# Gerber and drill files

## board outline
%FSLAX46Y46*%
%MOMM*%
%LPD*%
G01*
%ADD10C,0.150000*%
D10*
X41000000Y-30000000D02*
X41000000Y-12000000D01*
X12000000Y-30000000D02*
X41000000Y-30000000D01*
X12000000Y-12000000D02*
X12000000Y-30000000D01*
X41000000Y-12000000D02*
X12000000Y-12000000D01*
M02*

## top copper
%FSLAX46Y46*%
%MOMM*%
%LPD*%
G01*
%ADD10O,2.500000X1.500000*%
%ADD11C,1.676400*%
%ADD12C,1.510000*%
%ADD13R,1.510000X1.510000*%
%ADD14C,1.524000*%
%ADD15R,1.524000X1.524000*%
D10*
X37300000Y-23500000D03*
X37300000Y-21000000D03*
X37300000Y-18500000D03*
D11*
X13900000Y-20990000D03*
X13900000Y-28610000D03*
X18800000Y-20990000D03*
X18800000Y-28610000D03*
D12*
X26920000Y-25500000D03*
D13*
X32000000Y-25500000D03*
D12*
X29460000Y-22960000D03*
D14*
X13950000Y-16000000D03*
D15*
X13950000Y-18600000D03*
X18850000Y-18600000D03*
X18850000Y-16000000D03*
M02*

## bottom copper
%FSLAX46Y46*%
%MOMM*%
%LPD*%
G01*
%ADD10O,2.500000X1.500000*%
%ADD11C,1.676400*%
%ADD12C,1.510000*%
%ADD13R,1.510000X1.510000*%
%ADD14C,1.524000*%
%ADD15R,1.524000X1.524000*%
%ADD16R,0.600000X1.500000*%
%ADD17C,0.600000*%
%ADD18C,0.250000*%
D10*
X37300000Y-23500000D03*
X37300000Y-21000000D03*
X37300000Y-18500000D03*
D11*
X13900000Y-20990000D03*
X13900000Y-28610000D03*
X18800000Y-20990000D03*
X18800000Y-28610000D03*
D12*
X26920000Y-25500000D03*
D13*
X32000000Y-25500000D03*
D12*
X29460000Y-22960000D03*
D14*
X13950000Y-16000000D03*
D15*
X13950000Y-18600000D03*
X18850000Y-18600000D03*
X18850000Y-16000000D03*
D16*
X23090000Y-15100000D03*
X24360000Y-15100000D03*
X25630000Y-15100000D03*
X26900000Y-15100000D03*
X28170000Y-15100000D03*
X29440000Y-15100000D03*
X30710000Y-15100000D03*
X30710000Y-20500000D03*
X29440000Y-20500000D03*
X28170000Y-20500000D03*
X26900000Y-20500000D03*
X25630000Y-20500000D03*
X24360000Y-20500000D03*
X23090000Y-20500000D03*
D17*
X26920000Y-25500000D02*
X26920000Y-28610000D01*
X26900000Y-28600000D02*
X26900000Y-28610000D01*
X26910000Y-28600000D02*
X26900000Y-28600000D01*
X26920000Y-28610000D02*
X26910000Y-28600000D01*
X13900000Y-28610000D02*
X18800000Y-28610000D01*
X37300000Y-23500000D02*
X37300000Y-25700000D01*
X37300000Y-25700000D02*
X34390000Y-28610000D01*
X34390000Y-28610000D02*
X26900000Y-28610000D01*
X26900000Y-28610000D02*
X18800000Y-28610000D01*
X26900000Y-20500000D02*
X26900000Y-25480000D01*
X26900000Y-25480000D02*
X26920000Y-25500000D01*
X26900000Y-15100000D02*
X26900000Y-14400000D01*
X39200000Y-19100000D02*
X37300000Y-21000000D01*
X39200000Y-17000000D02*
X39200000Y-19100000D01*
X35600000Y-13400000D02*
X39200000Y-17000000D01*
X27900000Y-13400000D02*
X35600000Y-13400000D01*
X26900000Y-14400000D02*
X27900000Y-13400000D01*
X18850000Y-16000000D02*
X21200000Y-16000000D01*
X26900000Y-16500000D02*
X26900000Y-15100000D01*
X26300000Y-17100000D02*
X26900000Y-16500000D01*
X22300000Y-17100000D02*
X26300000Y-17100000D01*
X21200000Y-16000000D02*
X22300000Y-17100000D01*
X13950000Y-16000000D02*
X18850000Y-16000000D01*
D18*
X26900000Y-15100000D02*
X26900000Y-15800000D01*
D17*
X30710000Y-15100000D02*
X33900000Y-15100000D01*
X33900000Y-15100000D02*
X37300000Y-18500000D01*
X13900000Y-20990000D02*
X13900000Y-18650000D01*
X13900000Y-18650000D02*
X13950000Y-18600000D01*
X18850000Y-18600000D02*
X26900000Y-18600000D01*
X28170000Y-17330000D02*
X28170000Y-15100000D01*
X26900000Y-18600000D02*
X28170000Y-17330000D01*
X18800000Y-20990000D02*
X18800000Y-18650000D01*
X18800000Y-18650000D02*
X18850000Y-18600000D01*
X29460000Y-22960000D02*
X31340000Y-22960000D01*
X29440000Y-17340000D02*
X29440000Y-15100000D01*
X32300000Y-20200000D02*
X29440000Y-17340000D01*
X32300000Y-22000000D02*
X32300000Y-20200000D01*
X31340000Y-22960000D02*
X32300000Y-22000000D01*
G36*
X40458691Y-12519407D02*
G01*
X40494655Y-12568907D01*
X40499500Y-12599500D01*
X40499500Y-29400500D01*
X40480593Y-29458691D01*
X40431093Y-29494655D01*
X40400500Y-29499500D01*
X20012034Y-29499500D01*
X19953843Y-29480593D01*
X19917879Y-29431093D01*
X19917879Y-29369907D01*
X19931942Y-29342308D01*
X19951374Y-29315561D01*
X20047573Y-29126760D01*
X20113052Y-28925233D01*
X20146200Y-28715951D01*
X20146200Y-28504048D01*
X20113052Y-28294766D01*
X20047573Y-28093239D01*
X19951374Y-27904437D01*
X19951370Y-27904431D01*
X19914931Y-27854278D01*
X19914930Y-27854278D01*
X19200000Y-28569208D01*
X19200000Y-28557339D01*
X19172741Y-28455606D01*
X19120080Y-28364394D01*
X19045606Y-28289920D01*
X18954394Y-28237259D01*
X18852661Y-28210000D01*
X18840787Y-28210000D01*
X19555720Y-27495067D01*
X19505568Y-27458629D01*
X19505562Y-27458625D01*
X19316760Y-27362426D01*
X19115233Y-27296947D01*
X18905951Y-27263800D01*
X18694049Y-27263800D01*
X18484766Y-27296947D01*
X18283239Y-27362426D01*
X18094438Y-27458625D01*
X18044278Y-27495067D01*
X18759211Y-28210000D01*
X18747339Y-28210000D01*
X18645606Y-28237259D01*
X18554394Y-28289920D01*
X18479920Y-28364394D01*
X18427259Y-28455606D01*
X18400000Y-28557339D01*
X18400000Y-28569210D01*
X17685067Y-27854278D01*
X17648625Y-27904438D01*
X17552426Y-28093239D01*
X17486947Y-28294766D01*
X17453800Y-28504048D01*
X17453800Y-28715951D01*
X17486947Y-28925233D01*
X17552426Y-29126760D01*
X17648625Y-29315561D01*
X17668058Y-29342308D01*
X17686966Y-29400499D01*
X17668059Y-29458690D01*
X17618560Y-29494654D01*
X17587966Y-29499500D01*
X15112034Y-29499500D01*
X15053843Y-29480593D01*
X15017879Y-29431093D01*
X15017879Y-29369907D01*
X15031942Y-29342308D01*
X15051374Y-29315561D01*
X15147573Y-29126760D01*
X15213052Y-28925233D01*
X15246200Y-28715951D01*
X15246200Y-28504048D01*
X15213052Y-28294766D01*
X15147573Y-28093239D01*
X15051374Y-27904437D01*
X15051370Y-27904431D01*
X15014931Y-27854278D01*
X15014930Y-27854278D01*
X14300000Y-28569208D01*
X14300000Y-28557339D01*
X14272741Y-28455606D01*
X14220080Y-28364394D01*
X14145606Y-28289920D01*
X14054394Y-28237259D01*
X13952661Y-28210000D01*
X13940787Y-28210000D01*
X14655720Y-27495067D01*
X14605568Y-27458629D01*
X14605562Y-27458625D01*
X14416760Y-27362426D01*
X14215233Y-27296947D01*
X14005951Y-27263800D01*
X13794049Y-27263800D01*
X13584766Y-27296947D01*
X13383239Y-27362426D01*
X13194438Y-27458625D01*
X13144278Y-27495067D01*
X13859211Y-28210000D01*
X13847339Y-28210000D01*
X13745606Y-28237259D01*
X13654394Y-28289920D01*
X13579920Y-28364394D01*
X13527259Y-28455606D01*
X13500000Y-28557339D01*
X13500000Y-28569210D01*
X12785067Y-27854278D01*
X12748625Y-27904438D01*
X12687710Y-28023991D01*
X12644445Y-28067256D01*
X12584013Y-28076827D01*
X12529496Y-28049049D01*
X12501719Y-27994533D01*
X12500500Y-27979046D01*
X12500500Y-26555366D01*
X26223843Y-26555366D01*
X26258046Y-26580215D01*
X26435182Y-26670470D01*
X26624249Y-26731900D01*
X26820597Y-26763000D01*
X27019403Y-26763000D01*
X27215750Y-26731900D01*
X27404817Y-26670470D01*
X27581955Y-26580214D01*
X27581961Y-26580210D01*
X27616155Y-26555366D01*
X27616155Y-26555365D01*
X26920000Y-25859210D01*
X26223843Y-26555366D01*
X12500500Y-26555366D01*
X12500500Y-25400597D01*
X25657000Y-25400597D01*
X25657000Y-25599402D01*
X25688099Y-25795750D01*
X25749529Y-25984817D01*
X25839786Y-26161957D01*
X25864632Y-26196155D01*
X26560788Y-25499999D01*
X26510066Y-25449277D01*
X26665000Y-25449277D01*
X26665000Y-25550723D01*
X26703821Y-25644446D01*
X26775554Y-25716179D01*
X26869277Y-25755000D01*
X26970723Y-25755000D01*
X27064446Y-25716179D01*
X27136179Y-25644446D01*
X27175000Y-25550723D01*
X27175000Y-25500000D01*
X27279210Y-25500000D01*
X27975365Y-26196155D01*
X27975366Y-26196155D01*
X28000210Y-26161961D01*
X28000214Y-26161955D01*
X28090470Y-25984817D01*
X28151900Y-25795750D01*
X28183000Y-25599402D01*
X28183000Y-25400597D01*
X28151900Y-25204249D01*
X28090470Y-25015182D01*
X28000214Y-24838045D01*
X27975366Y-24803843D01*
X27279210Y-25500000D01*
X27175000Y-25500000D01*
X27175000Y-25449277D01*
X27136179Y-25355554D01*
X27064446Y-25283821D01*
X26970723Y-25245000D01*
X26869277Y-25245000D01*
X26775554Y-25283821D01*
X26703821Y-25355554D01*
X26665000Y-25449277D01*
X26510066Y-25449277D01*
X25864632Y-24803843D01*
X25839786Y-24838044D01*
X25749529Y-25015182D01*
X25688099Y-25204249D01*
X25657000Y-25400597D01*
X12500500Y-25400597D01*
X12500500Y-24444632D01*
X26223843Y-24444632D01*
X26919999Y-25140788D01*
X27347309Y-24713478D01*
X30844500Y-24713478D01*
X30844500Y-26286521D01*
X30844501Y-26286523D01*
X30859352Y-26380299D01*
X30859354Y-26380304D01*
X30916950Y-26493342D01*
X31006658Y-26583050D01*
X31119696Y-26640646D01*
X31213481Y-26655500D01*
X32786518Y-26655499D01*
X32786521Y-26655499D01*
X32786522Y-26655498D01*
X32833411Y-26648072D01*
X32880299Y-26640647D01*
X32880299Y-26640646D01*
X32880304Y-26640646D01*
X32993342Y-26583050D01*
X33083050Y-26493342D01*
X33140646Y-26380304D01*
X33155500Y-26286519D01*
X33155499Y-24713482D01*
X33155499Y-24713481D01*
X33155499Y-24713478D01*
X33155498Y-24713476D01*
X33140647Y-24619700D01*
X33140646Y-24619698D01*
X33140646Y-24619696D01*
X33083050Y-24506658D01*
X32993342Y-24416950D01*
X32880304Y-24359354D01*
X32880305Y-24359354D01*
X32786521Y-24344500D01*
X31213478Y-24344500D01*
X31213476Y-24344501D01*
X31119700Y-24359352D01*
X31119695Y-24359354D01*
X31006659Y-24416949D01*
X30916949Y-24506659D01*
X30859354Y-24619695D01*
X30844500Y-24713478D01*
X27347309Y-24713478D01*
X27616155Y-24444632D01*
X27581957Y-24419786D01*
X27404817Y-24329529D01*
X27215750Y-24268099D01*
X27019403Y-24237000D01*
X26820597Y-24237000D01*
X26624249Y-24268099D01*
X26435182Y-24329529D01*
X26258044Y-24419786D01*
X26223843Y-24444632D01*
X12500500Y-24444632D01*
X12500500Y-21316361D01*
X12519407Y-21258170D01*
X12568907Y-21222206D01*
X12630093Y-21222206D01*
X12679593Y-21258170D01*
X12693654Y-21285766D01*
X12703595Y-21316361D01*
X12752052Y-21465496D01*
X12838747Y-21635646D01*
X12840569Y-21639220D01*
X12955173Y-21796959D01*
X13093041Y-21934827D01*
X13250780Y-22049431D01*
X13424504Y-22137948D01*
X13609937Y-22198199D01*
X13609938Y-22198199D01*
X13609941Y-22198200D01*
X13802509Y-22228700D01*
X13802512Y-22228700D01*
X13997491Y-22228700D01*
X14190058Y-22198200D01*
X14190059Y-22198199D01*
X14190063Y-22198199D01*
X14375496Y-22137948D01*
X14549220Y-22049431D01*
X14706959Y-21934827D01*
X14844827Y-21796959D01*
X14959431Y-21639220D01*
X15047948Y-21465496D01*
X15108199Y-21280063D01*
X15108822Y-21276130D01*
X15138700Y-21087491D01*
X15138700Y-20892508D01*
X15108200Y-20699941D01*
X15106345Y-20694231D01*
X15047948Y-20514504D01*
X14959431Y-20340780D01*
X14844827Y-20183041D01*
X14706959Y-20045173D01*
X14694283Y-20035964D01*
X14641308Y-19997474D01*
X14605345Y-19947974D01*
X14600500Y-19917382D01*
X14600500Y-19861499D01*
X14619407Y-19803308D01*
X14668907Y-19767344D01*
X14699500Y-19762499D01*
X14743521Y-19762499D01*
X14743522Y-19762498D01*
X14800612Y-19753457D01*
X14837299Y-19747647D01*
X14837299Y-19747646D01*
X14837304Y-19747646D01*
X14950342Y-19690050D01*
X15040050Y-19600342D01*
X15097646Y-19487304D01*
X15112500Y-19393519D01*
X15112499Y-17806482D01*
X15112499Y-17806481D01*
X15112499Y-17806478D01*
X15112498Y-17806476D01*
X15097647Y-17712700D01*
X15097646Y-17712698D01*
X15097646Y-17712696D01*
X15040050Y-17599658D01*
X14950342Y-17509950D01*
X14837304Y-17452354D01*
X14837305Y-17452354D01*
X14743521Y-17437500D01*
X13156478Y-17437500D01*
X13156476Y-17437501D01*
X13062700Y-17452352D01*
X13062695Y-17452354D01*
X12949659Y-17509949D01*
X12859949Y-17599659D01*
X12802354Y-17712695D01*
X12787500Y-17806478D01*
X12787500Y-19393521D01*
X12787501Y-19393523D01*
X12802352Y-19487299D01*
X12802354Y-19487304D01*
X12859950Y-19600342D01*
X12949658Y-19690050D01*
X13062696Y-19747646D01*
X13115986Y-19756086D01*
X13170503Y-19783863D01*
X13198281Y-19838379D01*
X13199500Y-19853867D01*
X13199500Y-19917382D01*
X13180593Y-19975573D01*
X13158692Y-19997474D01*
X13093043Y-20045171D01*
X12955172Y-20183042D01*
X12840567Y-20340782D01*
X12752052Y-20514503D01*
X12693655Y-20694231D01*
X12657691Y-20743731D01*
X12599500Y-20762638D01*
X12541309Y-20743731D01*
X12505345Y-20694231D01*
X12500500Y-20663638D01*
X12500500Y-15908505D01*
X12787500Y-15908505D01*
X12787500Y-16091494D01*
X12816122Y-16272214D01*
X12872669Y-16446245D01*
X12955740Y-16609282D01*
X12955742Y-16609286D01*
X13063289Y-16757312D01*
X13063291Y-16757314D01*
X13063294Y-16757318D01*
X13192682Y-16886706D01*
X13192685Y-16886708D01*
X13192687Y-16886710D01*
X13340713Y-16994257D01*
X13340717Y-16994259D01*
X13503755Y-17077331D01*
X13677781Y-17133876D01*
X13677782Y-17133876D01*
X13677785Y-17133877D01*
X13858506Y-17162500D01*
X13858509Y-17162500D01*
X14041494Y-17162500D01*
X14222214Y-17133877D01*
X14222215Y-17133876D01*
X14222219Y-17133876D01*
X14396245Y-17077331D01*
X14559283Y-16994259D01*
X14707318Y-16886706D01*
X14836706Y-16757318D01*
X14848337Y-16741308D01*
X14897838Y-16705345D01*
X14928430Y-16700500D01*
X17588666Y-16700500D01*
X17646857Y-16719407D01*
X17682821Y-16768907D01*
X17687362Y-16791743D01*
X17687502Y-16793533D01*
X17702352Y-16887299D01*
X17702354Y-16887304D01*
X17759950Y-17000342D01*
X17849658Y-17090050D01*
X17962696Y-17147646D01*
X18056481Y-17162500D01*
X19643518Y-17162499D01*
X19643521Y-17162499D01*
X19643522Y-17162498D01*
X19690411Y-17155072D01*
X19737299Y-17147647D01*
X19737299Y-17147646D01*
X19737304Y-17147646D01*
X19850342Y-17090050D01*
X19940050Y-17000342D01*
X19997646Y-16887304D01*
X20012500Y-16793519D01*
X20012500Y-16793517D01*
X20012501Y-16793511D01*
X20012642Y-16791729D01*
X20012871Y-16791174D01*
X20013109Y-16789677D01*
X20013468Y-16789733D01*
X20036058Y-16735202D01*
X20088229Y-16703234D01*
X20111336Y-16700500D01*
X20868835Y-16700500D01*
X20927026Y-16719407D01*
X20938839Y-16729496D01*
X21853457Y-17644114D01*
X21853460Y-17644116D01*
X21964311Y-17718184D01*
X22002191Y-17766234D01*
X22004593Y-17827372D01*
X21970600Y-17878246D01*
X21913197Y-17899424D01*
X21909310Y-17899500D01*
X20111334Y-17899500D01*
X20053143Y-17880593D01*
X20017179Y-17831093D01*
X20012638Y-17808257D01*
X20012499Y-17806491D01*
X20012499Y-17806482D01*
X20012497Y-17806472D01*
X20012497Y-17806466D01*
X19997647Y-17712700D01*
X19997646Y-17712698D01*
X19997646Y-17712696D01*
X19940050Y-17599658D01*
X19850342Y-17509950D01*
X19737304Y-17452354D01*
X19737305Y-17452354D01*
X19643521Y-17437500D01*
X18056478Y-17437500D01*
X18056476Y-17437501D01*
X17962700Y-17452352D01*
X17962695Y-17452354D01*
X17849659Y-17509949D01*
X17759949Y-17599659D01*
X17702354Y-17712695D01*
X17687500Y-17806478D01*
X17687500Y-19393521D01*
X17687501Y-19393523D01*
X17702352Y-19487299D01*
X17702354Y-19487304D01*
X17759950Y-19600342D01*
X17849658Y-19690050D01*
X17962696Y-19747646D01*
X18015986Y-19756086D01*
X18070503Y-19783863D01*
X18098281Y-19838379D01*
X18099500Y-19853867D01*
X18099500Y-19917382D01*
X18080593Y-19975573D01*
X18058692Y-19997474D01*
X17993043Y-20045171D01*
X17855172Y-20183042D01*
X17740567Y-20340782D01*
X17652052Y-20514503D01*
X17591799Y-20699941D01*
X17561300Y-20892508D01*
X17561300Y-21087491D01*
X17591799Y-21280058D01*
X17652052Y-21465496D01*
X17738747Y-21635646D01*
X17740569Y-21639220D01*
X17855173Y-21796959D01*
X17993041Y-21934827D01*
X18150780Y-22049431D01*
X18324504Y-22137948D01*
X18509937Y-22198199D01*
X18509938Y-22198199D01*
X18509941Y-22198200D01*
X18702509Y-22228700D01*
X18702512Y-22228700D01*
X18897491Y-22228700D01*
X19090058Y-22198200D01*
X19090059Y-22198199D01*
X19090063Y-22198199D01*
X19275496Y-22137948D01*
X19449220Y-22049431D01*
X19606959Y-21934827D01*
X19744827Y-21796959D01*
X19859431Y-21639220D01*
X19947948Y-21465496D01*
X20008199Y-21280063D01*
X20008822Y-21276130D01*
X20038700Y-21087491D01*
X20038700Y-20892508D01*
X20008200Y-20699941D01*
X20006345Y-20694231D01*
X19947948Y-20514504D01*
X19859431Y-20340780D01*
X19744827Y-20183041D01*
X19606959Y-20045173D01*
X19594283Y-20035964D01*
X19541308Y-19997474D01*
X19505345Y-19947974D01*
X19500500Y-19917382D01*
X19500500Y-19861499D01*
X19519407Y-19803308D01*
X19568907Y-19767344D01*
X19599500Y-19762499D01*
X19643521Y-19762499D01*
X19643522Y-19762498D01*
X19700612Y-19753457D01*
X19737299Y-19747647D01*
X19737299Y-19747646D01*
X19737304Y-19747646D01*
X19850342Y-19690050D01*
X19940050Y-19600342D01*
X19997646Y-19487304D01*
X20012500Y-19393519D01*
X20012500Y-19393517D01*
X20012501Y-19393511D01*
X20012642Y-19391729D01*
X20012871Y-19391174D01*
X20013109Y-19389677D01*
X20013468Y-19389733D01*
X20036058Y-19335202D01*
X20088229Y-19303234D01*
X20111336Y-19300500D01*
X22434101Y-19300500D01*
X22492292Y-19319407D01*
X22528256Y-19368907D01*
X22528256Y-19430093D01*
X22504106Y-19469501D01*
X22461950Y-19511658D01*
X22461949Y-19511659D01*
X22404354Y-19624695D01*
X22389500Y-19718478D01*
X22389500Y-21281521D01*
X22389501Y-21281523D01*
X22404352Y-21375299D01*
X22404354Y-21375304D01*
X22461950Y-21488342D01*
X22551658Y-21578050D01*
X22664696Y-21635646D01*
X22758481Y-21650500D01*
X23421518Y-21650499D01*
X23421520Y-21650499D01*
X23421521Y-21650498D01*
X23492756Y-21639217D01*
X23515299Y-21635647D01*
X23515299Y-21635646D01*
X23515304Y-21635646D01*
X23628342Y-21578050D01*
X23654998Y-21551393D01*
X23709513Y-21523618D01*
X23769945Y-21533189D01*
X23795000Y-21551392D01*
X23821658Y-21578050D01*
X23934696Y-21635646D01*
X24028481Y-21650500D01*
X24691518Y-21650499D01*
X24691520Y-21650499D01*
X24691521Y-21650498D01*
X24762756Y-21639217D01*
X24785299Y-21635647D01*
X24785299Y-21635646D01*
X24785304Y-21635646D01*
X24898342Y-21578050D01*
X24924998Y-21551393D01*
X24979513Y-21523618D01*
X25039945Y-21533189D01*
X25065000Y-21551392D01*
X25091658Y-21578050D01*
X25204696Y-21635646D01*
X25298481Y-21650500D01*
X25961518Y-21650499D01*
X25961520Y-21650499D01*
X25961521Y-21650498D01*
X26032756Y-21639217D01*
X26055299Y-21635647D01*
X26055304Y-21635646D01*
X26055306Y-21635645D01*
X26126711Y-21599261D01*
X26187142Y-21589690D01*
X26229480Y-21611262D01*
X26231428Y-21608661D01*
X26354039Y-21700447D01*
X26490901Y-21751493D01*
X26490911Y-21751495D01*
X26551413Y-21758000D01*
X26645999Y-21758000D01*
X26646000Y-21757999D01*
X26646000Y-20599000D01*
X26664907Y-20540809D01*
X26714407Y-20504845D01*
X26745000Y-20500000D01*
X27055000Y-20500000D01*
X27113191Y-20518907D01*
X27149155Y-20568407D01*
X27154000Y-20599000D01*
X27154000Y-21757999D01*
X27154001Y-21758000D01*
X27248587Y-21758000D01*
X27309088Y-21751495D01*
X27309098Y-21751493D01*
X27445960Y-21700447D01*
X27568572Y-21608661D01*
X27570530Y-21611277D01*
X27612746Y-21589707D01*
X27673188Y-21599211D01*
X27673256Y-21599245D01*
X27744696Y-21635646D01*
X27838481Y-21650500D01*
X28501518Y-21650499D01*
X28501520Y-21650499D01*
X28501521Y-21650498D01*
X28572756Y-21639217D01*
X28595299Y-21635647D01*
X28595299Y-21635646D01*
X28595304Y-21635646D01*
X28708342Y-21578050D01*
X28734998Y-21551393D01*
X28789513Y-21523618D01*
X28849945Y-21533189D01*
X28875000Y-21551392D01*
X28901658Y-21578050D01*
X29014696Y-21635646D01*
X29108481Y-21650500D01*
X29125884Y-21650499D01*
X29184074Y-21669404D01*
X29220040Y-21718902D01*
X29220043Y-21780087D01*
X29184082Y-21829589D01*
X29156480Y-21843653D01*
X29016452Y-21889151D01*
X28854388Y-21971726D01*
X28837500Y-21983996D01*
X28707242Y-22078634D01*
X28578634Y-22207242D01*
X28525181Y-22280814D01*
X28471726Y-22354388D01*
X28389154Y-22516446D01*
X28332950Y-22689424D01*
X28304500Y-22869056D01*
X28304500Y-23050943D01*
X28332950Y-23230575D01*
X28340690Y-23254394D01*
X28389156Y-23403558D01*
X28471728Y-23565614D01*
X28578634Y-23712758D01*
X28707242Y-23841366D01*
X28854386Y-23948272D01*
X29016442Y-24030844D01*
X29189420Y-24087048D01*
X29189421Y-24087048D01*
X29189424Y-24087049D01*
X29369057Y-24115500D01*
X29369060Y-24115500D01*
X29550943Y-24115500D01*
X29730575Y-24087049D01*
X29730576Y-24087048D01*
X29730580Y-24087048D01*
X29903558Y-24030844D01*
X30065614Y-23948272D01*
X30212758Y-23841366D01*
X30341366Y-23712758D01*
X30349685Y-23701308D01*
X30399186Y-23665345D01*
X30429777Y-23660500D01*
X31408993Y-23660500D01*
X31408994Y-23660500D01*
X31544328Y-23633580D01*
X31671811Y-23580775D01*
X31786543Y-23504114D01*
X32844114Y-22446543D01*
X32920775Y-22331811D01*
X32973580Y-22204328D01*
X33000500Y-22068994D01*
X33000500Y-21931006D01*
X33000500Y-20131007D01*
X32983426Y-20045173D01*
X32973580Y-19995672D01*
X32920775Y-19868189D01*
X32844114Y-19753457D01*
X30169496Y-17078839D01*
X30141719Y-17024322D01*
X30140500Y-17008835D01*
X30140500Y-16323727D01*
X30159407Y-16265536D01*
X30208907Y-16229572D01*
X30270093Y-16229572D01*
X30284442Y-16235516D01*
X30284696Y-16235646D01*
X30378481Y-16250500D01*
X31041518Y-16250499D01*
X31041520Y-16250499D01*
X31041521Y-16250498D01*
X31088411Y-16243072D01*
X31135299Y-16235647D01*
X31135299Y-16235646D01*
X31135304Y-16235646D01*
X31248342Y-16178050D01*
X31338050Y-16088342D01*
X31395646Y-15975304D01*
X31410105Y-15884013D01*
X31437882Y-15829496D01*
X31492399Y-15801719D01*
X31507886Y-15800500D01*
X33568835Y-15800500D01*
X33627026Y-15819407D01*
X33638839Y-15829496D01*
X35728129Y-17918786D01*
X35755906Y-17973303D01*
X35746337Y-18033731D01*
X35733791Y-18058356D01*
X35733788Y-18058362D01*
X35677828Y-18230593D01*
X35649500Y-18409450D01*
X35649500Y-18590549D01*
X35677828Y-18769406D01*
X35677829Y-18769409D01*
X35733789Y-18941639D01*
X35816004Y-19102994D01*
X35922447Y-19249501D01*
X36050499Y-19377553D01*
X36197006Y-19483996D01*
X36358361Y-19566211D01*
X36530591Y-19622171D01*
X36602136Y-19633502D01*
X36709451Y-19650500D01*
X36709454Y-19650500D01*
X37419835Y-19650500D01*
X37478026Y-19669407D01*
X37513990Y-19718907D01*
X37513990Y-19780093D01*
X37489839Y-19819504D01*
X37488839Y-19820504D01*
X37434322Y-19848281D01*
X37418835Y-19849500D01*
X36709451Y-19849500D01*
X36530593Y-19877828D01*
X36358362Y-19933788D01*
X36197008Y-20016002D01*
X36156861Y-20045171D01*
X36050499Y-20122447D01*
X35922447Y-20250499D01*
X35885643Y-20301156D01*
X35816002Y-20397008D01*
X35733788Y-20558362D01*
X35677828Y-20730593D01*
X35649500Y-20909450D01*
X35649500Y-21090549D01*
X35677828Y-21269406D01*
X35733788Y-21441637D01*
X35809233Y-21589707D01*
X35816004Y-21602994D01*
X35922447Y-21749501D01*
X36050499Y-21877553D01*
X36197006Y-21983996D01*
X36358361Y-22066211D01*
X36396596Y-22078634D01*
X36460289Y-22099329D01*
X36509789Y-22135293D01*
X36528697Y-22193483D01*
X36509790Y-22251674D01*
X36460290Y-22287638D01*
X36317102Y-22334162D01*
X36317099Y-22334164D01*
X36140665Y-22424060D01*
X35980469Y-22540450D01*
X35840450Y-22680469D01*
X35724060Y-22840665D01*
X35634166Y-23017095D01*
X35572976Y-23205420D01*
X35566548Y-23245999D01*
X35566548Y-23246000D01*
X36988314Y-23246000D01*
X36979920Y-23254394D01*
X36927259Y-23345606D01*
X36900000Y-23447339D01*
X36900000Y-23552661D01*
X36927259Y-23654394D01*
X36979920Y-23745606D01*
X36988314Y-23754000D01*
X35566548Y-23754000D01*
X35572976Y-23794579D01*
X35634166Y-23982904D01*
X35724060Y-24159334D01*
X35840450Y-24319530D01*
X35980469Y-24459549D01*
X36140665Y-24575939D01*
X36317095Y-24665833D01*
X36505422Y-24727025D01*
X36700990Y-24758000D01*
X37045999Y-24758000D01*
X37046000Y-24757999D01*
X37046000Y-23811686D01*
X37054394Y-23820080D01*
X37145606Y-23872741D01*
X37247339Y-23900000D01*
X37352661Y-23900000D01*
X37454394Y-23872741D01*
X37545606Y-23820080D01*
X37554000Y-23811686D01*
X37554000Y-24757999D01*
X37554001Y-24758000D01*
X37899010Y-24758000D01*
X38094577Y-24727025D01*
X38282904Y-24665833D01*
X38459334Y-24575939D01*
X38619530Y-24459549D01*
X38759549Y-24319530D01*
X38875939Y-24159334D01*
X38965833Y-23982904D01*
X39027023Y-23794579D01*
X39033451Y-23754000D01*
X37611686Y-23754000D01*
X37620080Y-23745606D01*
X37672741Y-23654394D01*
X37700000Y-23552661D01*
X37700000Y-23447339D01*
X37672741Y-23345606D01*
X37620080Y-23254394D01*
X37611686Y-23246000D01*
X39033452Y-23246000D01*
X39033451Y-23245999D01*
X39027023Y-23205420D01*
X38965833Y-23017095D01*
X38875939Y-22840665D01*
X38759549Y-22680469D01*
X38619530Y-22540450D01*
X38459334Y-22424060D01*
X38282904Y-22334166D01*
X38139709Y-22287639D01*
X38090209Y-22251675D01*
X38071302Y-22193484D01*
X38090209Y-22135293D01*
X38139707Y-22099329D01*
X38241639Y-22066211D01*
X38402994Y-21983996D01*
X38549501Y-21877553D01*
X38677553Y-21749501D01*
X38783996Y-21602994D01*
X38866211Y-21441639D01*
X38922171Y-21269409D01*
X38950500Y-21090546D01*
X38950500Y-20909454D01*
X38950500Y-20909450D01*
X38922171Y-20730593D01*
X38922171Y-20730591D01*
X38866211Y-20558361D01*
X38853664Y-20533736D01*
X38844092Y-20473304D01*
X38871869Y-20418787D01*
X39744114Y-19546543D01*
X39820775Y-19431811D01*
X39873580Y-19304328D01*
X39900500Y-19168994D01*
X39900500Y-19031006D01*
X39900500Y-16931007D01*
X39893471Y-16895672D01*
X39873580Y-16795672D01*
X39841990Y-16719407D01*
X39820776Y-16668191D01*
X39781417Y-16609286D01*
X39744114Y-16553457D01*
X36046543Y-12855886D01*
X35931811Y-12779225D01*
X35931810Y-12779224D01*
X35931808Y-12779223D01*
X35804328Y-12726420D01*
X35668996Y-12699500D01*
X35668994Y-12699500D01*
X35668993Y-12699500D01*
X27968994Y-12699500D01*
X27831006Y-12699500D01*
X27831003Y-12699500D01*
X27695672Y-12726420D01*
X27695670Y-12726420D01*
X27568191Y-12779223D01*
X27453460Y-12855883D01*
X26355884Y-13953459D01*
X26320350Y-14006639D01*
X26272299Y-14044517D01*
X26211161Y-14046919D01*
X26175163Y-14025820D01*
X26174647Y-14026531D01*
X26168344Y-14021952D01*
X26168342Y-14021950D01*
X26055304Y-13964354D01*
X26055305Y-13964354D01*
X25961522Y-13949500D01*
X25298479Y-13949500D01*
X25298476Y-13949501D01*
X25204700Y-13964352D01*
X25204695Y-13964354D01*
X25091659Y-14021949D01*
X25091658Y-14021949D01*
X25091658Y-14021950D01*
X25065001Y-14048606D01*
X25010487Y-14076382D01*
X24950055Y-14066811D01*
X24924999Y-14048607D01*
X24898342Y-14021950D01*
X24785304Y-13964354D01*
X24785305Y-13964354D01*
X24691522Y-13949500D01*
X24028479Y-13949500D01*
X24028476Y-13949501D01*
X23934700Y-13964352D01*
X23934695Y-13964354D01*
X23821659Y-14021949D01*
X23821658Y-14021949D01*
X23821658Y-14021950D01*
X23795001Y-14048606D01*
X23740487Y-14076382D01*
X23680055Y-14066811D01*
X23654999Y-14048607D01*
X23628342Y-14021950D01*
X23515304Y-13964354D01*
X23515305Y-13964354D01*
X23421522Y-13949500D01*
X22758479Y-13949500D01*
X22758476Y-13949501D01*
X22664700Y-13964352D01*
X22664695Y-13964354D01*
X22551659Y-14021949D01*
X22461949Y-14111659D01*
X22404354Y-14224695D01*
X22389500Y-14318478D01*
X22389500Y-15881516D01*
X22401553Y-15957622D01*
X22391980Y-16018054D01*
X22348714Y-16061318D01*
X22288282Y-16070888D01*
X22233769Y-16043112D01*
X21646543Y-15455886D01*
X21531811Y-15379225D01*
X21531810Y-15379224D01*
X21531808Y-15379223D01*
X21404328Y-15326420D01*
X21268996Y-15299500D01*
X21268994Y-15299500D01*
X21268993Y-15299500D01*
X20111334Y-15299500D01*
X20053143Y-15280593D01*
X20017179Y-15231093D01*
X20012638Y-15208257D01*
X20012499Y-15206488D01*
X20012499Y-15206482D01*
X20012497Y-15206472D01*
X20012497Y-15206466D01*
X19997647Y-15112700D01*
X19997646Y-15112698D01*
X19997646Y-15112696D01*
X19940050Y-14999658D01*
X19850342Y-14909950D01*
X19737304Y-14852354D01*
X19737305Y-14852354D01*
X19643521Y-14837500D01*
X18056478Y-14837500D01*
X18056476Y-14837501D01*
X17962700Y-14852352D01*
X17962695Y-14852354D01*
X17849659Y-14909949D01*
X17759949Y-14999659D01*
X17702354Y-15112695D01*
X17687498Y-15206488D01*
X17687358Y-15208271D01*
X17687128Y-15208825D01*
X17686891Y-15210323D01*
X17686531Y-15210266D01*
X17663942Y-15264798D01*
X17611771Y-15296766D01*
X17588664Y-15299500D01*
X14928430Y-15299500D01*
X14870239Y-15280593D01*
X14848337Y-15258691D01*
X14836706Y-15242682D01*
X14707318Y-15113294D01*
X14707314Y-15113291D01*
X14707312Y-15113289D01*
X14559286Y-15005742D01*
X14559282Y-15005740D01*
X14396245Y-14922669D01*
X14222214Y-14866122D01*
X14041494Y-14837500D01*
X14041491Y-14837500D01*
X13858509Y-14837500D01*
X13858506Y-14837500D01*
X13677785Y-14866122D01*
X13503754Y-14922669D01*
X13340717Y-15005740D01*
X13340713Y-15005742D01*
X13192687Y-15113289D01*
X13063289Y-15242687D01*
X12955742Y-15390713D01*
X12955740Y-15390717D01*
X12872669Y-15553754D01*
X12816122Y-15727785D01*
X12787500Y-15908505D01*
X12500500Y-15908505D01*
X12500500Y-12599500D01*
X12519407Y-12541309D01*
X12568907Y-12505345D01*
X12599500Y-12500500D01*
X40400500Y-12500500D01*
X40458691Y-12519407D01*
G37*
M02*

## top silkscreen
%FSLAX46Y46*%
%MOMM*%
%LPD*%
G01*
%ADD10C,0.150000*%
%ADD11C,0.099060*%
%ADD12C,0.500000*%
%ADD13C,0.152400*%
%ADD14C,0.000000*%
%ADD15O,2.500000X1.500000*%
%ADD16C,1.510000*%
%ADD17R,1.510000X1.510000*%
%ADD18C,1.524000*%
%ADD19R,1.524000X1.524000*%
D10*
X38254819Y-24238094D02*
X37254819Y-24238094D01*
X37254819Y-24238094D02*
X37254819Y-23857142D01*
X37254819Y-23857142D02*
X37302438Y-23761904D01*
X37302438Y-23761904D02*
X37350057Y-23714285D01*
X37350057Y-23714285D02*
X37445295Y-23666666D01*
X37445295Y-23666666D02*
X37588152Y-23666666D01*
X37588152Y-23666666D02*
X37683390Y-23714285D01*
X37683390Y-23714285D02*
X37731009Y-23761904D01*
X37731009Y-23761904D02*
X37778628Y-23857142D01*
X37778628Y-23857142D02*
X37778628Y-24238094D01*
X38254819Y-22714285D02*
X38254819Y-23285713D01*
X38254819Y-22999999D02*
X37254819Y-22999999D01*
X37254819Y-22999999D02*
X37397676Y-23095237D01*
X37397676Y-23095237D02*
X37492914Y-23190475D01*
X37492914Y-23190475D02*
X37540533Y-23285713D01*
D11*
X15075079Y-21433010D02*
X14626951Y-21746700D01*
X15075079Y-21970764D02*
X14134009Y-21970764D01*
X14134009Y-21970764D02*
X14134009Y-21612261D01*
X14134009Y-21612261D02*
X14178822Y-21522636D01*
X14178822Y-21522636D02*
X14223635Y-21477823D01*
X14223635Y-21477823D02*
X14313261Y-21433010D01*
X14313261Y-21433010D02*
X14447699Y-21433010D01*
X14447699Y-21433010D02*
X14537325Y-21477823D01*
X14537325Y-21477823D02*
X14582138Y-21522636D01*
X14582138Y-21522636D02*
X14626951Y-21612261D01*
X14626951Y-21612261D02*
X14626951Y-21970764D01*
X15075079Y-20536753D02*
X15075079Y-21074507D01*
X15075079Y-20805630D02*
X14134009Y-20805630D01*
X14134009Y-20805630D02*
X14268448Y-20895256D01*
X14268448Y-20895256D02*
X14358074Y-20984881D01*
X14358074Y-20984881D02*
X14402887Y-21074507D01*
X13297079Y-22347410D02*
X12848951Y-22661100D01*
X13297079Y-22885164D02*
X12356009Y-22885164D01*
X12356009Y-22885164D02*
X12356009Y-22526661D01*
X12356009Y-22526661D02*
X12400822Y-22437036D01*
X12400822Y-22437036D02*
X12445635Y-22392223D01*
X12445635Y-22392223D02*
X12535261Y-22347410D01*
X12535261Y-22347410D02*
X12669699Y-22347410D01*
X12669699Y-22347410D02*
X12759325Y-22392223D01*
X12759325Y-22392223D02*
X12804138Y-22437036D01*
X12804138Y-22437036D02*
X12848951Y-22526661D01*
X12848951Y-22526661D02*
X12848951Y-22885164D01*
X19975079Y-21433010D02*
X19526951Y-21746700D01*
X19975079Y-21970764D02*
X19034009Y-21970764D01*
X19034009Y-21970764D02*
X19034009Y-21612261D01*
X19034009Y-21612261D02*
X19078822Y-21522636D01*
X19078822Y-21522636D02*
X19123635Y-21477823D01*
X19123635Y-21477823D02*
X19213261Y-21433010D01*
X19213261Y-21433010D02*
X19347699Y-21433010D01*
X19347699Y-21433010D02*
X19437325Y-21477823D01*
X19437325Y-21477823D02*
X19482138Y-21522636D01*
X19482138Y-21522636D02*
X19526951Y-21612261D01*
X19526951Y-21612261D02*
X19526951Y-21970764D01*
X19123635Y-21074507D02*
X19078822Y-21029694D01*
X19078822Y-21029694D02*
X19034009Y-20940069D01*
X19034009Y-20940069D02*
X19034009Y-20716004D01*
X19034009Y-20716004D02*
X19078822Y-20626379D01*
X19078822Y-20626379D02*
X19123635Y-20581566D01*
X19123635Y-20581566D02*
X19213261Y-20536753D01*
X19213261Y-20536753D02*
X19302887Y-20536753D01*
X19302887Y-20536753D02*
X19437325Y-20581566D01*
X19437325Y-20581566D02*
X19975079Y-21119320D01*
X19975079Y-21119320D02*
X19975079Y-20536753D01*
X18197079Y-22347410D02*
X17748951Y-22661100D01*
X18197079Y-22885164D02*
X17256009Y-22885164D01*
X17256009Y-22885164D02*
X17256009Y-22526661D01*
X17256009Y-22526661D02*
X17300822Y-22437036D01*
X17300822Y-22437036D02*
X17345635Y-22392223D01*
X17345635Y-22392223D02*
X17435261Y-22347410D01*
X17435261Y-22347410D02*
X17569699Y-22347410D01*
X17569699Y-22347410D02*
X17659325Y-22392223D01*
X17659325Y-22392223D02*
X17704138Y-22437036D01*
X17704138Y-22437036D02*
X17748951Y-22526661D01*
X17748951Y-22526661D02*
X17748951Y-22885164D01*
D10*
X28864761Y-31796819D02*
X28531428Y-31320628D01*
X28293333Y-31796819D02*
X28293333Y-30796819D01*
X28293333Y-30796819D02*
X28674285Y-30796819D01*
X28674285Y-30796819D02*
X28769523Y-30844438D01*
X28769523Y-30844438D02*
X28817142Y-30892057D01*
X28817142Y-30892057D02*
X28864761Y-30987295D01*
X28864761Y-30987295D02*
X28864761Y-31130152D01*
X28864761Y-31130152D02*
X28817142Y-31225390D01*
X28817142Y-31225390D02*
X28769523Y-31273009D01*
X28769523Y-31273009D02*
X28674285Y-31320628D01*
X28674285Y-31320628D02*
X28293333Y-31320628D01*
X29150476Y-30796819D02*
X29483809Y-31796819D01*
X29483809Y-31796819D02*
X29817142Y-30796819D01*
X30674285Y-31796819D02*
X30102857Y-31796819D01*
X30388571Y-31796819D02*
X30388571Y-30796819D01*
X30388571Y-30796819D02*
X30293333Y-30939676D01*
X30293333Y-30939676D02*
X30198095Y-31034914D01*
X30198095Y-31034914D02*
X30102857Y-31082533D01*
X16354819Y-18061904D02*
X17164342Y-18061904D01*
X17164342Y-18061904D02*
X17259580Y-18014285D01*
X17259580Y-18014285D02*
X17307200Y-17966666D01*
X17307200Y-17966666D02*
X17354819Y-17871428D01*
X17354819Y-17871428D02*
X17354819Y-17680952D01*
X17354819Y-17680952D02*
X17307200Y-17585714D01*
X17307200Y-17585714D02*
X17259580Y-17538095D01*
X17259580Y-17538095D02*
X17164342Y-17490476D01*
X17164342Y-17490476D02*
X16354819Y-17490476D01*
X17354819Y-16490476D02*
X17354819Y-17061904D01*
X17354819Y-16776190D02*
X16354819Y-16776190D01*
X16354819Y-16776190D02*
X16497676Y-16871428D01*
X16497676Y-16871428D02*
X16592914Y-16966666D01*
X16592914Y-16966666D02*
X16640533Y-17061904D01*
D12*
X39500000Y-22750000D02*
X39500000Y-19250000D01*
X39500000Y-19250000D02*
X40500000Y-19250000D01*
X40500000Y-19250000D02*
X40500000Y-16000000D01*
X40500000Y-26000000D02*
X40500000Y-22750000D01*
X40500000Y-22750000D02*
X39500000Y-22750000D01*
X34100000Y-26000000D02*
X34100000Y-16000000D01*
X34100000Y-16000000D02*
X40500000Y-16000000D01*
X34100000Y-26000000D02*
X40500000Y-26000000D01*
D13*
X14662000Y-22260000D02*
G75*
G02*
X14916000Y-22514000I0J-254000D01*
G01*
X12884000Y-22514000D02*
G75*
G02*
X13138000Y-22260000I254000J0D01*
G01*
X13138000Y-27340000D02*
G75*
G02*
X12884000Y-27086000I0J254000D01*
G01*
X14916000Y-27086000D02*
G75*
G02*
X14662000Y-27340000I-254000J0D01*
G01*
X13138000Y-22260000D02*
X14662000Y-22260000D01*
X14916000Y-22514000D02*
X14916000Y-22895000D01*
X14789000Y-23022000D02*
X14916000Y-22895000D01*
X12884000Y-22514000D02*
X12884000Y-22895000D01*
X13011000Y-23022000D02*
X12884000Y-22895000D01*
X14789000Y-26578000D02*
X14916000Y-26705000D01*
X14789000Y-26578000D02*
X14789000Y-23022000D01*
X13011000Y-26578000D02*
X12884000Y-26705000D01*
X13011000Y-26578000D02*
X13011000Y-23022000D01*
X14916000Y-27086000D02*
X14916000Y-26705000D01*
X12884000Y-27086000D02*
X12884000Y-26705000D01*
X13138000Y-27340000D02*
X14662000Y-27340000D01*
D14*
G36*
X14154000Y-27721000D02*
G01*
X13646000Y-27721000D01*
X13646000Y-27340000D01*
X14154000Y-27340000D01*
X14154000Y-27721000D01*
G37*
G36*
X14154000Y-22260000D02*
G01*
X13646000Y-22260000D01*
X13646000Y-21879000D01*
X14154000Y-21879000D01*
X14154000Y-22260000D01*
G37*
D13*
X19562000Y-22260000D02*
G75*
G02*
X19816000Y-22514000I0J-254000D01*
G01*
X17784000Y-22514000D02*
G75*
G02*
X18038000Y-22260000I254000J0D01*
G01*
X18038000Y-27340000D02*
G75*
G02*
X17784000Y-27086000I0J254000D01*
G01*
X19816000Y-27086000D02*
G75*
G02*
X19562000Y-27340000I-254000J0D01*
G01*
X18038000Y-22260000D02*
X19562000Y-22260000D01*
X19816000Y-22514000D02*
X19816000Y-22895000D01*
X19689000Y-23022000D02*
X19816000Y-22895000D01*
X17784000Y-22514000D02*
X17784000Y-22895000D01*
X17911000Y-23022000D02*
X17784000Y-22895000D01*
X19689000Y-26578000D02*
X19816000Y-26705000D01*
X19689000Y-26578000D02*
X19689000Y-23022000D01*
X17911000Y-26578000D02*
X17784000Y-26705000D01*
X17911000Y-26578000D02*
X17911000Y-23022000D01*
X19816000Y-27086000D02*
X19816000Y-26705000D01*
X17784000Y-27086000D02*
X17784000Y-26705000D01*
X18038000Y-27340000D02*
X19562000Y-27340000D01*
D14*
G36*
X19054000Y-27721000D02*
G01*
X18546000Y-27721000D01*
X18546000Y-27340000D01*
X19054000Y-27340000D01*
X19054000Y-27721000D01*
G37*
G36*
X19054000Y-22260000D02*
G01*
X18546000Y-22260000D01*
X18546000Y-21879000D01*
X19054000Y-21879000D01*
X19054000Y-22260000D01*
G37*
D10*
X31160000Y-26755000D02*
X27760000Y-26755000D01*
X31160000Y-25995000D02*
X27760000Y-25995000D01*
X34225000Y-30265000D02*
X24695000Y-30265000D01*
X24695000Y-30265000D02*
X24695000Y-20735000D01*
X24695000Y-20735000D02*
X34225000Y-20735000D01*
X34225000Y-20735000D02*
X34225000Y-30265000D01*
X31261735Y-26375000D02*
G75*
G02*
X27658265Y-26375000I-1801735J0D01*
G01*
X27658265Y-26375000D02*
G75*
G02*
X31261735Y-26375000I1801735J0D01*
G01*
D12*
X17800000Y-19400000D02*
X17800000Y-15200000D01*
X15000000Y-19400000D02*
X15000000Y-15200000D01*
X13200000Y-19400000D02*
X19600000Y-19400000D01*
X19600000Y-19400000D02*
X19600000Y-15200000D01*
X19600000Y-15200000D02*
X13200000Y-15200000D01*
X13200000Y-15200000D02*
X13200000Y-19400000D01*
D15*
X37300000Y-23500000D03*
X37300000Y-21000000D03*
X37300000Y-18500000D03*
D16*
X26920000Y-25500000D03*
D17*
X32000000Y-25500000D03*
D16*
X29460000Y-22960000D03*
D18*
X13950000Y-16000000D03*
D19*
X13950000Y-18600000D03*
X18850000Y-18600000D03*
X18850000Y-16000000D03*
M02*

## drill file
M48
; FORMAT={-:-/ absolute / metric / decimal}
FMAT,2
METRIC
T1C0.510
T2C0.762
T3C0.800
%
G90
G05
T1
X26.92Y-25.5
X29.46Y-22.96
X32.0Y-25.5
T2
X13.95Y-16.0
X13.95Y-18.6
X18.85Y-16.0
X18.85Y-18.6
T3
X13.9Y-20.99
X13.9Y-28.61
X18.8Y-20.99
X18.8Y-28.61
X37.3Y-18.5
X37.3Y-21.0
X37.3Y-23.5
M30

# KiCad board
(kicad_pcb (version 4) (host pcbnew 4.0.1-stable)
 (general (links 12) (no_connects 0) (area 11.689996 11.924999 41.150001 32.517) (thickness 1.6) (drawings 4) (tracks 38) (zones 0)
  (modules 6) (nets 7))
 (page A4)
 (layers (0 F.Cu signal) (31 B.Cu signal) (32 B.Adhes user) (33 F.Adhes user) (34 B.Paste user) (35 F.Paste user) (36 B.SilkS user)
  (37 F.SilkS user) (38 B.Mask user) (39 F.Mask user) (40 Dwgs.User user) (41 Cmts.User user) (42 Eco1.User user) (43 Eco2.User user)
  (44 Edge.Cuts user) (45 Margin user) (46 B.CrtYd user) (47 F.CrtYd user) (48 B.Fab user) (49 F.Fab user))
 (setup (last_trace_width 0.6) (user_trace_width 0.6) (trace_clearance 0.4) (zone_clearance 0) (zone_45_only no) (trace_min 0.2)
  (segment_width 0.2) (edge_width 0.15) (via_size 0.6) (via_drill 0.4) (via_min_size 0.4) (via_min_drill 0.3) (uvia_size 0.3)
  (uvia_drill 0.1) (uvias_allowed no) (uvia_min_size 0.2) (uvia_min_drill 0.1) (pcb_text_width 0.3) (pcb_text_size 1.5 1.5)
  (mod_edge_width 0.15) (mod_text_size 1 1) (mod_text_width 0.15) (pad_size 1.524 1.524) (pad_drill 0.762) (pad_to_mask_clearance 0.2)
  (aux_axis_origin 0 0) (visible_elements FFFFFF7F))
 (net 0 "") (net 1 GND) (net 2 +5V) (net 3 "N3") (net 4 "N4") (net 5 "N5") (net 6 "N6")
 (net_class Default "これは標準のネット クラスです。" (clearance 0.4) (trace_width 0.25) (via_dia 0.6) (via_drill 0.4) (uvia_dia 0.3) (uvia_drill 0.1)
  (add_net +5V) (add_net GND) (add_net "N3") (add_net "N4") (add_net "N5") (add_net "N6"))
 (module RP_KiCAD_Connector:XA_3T (layer F.Cu) (at 37.3 23.5 90)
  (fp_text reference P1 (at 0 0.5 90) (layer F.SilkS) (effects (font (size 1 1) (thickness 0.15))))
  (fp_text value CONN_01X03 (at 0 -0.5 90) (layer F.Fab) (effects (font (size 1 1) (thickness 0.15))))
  (fp_line (start 0.75 2.2) (end 4.25 2.2) (layer F.SilkS) (width 0.5))
  (fp_line (start 4.25 2.2) (end 4.25 3.2) (layer F.SilkS) (width 0.5))
  (fp_line (start 4.25 3.2) (end 7.5 3.2) (layer F.SilkS) (width 0.5))
  (fp_line (start -2.5 3.2) (end 0.75 3.2) (layer F.SilkS) (width 0.5))
  (fp_line (start 0.75 3.2) (end 0.75 2.2) (layer F.SilkS) (width 0.5))
  (fp_line (start -2.5 -3.2) (end 7.5 -3.2) (layer F.SilkS) (width 0.5))
  (fp_line (start 7.5 -3.2) (end 7.5 3.2) (layer F.SilkS) (width 0.5))
  (fp_line (start -2.5 -3.2) (end -2.5 3.2) (layer F.SilkS) (width 0.5))
  (pad 1 thru_hole oval (at 0 0 90) (size 1.5 2.5) (drill 0.8) (layers *.Cu *.Mask F.SilkS) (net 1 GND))
  (pad 2 thru_hole oval (at 2.5 0 90) (size 1.5 2.5) (drill 0.8) (layers *.Cu *.Mask F.SilkS) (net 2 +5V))
  (pad 3 thru_hole oval (at 5 0 90) (size 1.5 2.5) (drill 0.8) (layers *.Cu *.Mask F.SilkS) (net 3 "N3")))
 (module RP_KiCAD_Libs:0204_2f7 (layer F.Cu) (at 13.9 24.8 270)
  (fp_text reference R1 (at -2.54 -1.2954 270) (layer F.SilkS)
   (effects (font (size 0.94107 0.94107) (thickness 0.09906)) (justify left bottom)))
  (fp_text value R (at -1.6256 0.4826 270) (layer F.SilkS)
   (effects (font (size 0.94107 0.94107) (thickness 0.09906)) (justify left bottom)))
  (fp_arc (start -2.286 -0.762) (end -2.54 -0.762) (angle 90) (layer F.SilkS) (width 0.1524))
  (fp_arc (start -2.286 0.762) (end -2.54 0.762) (angle -90) (layer F.SilkS) (width 0.1524))
  (fp_arc (start 2.286 0.762) (end 2.286 1.016) (angle -90) (layer F.SilkS) (width 0.1524))
  (fp_arc (start 2.286 -0.762) (end 2.286 -1.016) (angle 90) (layer F.SilkS) (width 0.1524))
  (fp_line (start -2.54 0.762) (end -2.54 -0.762) (layer F.SilkS) (width 0.1524))
  (fp_line (start -2.286 -1.016) (end -1.905 -1.016) (layer F.SilkS) (width 0.1524))
  (fp_line (start -1.778 -0.889) (end -1.905 -1.016) (layer F.SilkS) (width 0.1524))
  (fp_line (start -2.286 1.016) (end -1.905 1.016) (layer F.SilkS) (width 0.1524))
  (fp_line (start -1.778 0.889) (end -1.905 1.016) (layer F.SilkS) (width 0.1524))
  (fp_line (start 1.778 -0.889) (end 1.905 -1.016) (layer F.SilkS) (width 0.1524))
  (fp_line (start 1.778 -0.889) (end -1.778 -0.889) (layer F.SilkS) (width 0.1524))
  (fp_line (start 1.778 0.889) (end 1.905 1.016) (layer F.SilkS) (width 0.1524))
  (fp_line (start 1.778 0.889) (end -1.778 0.889) (layer F.SilkS) (width 0.1524))
  (fp_line (start 2.286 -1.016) (end 1.905 -1.016) (layer F.SilkS) (width 0.1524))
  (fp_line (start 2.286 1.016) (end 1.905 1.016) (layer F.SilkS) (width 0.1524))
  (fp_line (start 2.54 0.762) (end 2.54 -0.762) (layer F.SilkS) (width 0.1524))
  (fp_poly (pts (xy 2.54 0.254) (xy 2.921 0.254) (xy 2.921 -0.254) (xy 2.54 -0.254)) (layer F.SilkS) (width 0))
  (fp_poly (pts (xy -2.921 0.254) (xy -2.54 0.254) (xy -2.54 -0.254) (xy -2.921 -0.254)) (layer F.SilkS) (width 0))
  (pad 1 thru_hole circle (at -3.81 0 270) (size 1.6764 1.6764) (drill 0.8) (layers *.Cu *.Mask) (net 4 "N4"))
  (pad 2 thru_hole circle (at 3.81 0 270) (size 1.6764 1.6764) (drill 0.8) (layers *.Cu *.Mask) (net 1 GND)))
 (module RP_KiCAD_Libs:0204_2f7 (layer F.Cu) (at 18.8 24.8 270)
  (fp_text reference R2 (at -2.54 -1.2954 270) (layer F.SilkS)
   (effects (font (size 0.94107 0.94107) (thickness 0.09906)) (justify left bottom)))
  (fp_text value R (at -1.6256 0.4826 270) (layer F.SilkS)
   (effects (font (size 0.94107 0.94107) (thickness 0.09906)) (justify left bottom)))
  (fp_arc (start -2.286 -0.762) (end -2.54 -0.762) (angle 90) (layer F.SilkS) (width 0.1524))
  (fp_arc (start -2.286 0.762) (end -2.54 0.762) (angle -90) (layer F.SilkS) (width 0.1524))
  (fp_arc (start 2.286 0.762) (end 2.286 1.016) (angle -90) (layer F.SilkS) (width 0.1524))
  (fp_arc (start 2.286 -0.762) (end 2.286 -1.016) (angle 90) (layer F.SilkS) (width 0.1524))
  (fp_line (start -2.54 0.762) (end -2.54 -0.762) (layer F.SilkS) (width 0.1524))
  (fp_line (start -2.286 -1.016) (end -1.905 -1.016) (layer F.SilkS) (width 0.1524))
  (fp_line (start -1.778 -0.889) (end -1.905 -1.016) (layer F.SilkS) (width 0.1524))
  (fp_line (start -2.286 1.016) (end -1.905 1.016) (layer F.SilkS) (width 0.1524))
  (fp_line (start -1.778 0.889) (end -1.905 1.016) (layer F.SilkS) (width 0.1524))
  (fp_line (start 1.778 -0.889) (end 1.905 -1.016) (layer F.SilkS) (width 0.1524))
  (fp_line (start 1.778 -0.889) (end -1.778 -0.889) (layer F.SilkS) (width 0.1524))
  (fp_line (start 1.778 0.889) (end 1.905 1.016) (layer F.SilkS) (width 0.1524))
  (fp_line (start 1.778 0.889) (end -1.778 0.889) (layer F.SilkS) (width 0.1524))
  (fp_line (start 2.286 -1.016) (end 1.905 -1.016) (layer F.SilkS) (width 0.1524))
  (fp_line (start 2.286 1.016) (end 1.905 1.016) (layer F.SilkS) (width 0.1524))
  (fp_line (start 2.54 0.762) (end 2.54 -0.762) (layer F.SilkS) (width 0.1524))
  (fp_poly (pts (xy 2.54 0.254) (xy 2.921 0.254) (xy 2.921 -0.254) (xy 2.54 -0.254)) (layer F.SilkS) (width 0))
  (fp_poly (pts (xy -2.921 0.254) (xy -2.54 0.254) (xy -2.54 -0.254) (xy -2.921 -0.254)) (layer F.SilkS) (width 0))
  (pad 1 thru_hole circle (at -3.81 0 270) (size 1.6764 1.6764) (drill 0.8) (layers *.Cu *.Mask) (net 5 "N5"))
  (pad 2 thru_hole circle (at 3.81 0 270) (size 1.6764 1.6764) (drill 0.8) (layers *.Cu *.Mask) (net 1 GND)))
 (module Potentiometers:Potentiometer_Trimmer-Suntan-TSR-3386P (layer F.Cu) (at 32 25.5 180)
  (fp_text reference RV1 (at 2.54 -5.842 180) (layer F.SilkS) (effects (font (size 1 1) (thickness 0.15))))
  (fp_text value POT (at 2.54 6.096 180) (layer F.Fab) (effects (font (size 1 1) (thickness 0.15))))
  (fp_line (start 0.84 -1.255) (end 4.24 -1.255) (layer F.SilkS) (width 0.15))
  (fp_line (start 0.84 -0.495) (end 4.24 -0.495) (layer F.SilkS) (width 0.15))
  (fp_line (start -2.225 -4.765) (end 7.305 -4.765) (layer F.SilkS) (width 0.15))
  (fp_line (start 7.305 -4.765) (end 7.305 4.765) (layer F.SilkS) (width 0.15))
  (fp_line (start 7.305 4.765) (end -2.225 4.765) (layer F.SilkS) (width 0.15))
  (fp_line (start -2.225 4.765) (end -2.225 -4.765) (layer F.SilkS) (width 0.15))
  (fp_circle (center 2.54 -0.875) (end 4.115 0) (layer F.SilkS) (width 0.15))
  (pad 3 thru_hole circle (at 5.08 0 180) (size 1.51 1.51) (drill 0.51) (layers *.Cu *.Mask F.SilkS) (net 1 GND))
  (pad 1 thru_hole rect (at 0 0 180) (size 1.51 1.51) (drill 0.51) (layers *.Cu *.Mask F.SilkS))
  (pad 2 thru_hole circle (at 2.54 2.54 180) (size 1.51 1.51) (drill 0.51) (layers *.Cu *.Mask F.SilkS) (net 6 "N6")))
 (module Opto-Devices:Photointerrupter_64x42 (layer F.Cu) (at 16.4 17.3 90)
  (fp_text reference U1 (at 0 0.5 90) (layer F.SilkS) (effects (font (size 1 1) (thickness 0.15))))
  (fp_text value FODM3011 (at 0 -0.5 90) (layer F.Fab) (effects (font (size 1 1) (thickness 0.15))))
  (fp_line (start -2.1 1.4) (end 2.1 1.4) (layer F.SilkS) (width 0.5))
  (fp_line (start -2.1 -1.4) (end 2.1 -1.4) (layer F.SilkS) (width 0.5))
  (fp_line (start -2.1 -3.2) (end -2.1 3.2) (layer F.SilkS) (width 0.5))
  (fp_line (start -2.1 3.2) (end 2.1 3.2) (layer F.SilkS) (width 0.5))
  (fp_line (start 2.1 3.2) (end 2.1 -3.2) (layer F.SilkS) (width 0.5))
  (fp_line (start 2.1 -3.2) (end -2.1 -3.2) (layer F.SilkS) (width 0.5))
  (pad 1 thru_hole circle (at 1.3 -2.45 90) (size 1.524 1.524) (drill 0.762) (layers *.Cu *.Mask F.SilkS) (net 2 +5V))
  (pad 2 thru_hole rect (at -1.3 -2.45 90) (size 1.524 1.524) (drill 0.762) (layers *.Cu *.Mask F.SilkS) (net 4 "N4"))
  (pad 3 thru_hole rect (at -1.3 2.45 90) (size 1.524 1.524) (drill 0.762) (layers *.Cu *.Mask F.SilkS) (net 5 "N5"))
  (pad 4 thru_hole rect (at 1.3 2.45 90) (size 1.524 1.524) (drill 0.762) (layers *.Cu *.Mask F.SilkS) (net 2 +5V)))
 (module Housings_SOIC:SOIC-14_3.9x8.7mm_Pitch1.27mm (layer B.Cu) (at 26.9 17.8 270)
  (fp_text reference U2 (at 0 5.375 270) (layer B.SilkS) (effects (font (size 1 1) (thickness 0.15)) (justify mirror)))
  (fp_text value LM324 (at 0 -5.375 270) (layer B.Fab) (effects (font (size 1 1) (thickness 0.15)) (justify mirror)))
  (pad 1 smd rect (at -2.7 3.81 270) (size 1.5 0.6) (layers B.Cu B.Paste B.Mask))
  (pad 2 smd rect (at -2.7 2.54 270) (size 1.5 0.6) (layers B.Cu B.Paste B.Mask))
  (pad 3 smd rect (at -2.7 1.27 270) (size 1.5 0.6) (layers B.Cu B.Paste B.Mask))
  (pad 4 smd rect (at -2.7 0 270) (size 1.5 0.6) (layers B.Cu B.Paste B.Mask) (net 2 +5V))
  (pad 5 smd rect (at -2.7 -1.27 270) (size 1.5 0.6) (layers B.Cu B.Paste B.Mask) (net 5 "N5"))
  (pad 6 smd rect (at -2.7 -2.54 270) (size 1.5 0.6) (layers B.Cu B.Paste B.Mask) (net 6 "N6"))
  (pad 7 smd rect (at -2.7 -3.81 270) (size 1.5 0.6) (layers B.Cu B.Paste B.Mask) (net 3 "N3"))
  (pad 8 smd rect (at 2.7 -3.81 270) (size 1.5 0.6) (layers B.Cu B.Paste B.Mask))
  (pad 9 smd rect (at 2.7 -2.54 270) (size 1.5 0.6) (layers B.Cu B.Paste B.Mask))
  (pad 10 smd rect (at 2.7 -1.27 270) (size 1.5 0.6) (layers B.Cu B.Paste B.Mask))
  (pad 11 smd rect (at 2.7 0 270) (size 1.5 0.6) (layers B.Cu B.Paste B.Mask) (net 1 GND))
  (pad 12 smd rect (at 2.7 1.27 270) (size 1.5 0.6) (layers B.Cu B.Paste B.Mask))
  (pad 13 smd rect (at 2.7 2.54 270) (size 1.5 0.6) (layers B.Cu B.Paste B.Mask))
  (pad 14 smd rect (at 2.7 3.81 270) (size 1.5 0.6) (layers B.Cu B.Paste B.Mask)))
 (gr_line (start 41 30) (end 41 12) (angle 90) (layer Edge.Cuts) (width 0.15))
 (gr_line (start 12 30) (end 41 30) (angle 90) (layer Edge.Cuts) (width 0.15))
 (gr_line (start 12 12) (end 12 30) (angle 90) (layer Edge.Cuts) (width 0.15))
 (gr_line (start 41 12) (end 12 12) (angle 90) (layer Edge.Cuts) (width 0.15))
 (segment (start 26.92 25.5) (end 26.92 28.61) (width 0.6) (layer B.Cu) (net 1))
 (segment (start 26.9 28.6) (end 26.9 28.61) (width 0.6) (layer B.Cu) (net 1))
 (segment (start 26.91 28.6) (end 26.9 28.6) (width 0.6) (layer B.Cu) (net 1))
 (segment (start 26.92 28.61) (end 26.91 28.6) (width 0.6) (layer B.Cu) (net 1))
 (segment (start 13.9 28.61) (end 18.8 28.61) (width 0.6) (layer B.Cu) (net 1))
 (segment (start 37.3 23.5) (end 37.3 25.7) (width 0.6) (layer B.Cu) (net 1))
 (segment (start 37.3 25.7) (end 34.39 28.61) (width 0.6) (layer B.Cu) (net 1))
 (segment (start 34.39 28.61) (end 26.9 28.61) (width 0.6) (layer B.Cu) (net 1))
 (segment (start 26.9 28.61) (end 18.8 28.61) (width 0.6) (layer B.Cu) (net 1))
 (segment (start 26.9 20.5) (end 26.9 25.48) (width 0.6) (layer B.Cu) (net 1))
 (segment (start 26.9 25.48) (end 26.92 25.5) (width 0.6) (layer B.Cu) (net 1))
 (segment (start 26.9 15.1) (end 26.9 14.4) (width 0.6) (layer B.Cu) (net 2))
 (segment (start 39.2 19.1) (end 37.3 21) (width 0.6) (layer B.Cu) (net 2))
 (segment (start 39.2 17) (end 39.2 19.1) (width 0.6) (layer B.Cu) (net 2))
 (segment (start 35.6 13.4) (end 39.2 17) (width 0.6) (layer B.Cu) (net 2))
 (segment (start 27.9 13.4) (end 35.6 13.4) (width 0.6) (layer B.Cu) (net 2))
 (segment (start 26.9 14.4) (end 27.9 13.4) (width 0.6) (layer B.Cu) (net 2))
 (segment (start 18.85 16) (end 21.2 16) (width 0.6) (layer B.Cu) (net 2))
 (segment (start 26.9 16.5) (end 26.9 15.1) (width 0.6) (layer B.Cu) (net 2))
 (segment (start 26.3 17.1) (end 26.9 16.5) (width 0.6) (layer B.Cu) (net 2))
 (segment (start 22.3 17.1) (end 26.3 17.1) (width 0.6) (layer B.Cu) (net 2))
 (segment (start 21.2 16) (end 22.3 17.1) (width 0.6) (layer B.Cu) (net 2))
 (segment (start 13.95 16) (end 18.85 16) (width 0.6) (layer B.Cu) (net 2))
 (segment (start 26.9 15.1) (end 26.9 15.8) (width 0.25) (layer B.Cu) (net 2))
 (segment (start 30.71 15.1) (end 33.9 15.1) (width 0.6) (layer B.Cu) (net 3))
 (segment (start 33.9 15.1) (end 37.3 18.5) (width 0.6) (layer B.Cu) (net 3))
 (segment (start 13.9 20.99) (end 13.9 18.65) (width 0.6) (layer B.Cu) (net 4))
 (segment (start 13.9 18.65) (end 13.95 18.6) (width 0.6) (layer B.Cu) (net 4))
 (segment (start 18.85 18.6) (end 26.9 18.6) (width 0.6) (layer B.Cu) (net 5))
 (segment (start 28.17 17.33) (end 28.17 15.1) (width 0.6) (layer B.Cu) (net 5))
 (segment (start 26.9 18.6) (end 28.17 17.33) (width 0.6) (layer B.Cu) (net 5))
 (segment (start 18.8 20.99) (end 18.8 18.65) (width 0.6) (layer B.Cu) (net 5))
 (segment (start 18.8 18.65) (end 18.85 18.6) (width 0.6) (layer B.Cu) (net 5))
 (segment (start 29.46 22.96) (end 31.34 22.96) (width 0.6) (layer B.Cu) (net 6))
 (segment (start 29.44 17.34) (end 29.44 15.1) (width 0.6) (layer B.Cu) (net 6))
 (segment (start 32.3 20.2) (end 29.44 17.34) (width 0.6) (layer B.Cu) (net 6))
 (segment (start 32.3 22) (end 32.3 20.2) (width 0.6) (layer B.Cu) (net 6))
 (segment (start 31.34 22.96) (end 32.3 22) (width 0.6) (layer B.Cu) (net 6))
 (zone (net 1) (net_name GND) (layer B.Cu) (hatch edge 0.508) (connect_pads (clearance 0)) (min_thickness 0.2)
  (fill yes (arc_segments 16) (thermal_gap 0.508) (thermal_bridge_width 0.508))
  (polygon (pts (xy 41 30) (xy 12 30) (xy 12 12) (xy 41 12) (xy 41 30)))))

